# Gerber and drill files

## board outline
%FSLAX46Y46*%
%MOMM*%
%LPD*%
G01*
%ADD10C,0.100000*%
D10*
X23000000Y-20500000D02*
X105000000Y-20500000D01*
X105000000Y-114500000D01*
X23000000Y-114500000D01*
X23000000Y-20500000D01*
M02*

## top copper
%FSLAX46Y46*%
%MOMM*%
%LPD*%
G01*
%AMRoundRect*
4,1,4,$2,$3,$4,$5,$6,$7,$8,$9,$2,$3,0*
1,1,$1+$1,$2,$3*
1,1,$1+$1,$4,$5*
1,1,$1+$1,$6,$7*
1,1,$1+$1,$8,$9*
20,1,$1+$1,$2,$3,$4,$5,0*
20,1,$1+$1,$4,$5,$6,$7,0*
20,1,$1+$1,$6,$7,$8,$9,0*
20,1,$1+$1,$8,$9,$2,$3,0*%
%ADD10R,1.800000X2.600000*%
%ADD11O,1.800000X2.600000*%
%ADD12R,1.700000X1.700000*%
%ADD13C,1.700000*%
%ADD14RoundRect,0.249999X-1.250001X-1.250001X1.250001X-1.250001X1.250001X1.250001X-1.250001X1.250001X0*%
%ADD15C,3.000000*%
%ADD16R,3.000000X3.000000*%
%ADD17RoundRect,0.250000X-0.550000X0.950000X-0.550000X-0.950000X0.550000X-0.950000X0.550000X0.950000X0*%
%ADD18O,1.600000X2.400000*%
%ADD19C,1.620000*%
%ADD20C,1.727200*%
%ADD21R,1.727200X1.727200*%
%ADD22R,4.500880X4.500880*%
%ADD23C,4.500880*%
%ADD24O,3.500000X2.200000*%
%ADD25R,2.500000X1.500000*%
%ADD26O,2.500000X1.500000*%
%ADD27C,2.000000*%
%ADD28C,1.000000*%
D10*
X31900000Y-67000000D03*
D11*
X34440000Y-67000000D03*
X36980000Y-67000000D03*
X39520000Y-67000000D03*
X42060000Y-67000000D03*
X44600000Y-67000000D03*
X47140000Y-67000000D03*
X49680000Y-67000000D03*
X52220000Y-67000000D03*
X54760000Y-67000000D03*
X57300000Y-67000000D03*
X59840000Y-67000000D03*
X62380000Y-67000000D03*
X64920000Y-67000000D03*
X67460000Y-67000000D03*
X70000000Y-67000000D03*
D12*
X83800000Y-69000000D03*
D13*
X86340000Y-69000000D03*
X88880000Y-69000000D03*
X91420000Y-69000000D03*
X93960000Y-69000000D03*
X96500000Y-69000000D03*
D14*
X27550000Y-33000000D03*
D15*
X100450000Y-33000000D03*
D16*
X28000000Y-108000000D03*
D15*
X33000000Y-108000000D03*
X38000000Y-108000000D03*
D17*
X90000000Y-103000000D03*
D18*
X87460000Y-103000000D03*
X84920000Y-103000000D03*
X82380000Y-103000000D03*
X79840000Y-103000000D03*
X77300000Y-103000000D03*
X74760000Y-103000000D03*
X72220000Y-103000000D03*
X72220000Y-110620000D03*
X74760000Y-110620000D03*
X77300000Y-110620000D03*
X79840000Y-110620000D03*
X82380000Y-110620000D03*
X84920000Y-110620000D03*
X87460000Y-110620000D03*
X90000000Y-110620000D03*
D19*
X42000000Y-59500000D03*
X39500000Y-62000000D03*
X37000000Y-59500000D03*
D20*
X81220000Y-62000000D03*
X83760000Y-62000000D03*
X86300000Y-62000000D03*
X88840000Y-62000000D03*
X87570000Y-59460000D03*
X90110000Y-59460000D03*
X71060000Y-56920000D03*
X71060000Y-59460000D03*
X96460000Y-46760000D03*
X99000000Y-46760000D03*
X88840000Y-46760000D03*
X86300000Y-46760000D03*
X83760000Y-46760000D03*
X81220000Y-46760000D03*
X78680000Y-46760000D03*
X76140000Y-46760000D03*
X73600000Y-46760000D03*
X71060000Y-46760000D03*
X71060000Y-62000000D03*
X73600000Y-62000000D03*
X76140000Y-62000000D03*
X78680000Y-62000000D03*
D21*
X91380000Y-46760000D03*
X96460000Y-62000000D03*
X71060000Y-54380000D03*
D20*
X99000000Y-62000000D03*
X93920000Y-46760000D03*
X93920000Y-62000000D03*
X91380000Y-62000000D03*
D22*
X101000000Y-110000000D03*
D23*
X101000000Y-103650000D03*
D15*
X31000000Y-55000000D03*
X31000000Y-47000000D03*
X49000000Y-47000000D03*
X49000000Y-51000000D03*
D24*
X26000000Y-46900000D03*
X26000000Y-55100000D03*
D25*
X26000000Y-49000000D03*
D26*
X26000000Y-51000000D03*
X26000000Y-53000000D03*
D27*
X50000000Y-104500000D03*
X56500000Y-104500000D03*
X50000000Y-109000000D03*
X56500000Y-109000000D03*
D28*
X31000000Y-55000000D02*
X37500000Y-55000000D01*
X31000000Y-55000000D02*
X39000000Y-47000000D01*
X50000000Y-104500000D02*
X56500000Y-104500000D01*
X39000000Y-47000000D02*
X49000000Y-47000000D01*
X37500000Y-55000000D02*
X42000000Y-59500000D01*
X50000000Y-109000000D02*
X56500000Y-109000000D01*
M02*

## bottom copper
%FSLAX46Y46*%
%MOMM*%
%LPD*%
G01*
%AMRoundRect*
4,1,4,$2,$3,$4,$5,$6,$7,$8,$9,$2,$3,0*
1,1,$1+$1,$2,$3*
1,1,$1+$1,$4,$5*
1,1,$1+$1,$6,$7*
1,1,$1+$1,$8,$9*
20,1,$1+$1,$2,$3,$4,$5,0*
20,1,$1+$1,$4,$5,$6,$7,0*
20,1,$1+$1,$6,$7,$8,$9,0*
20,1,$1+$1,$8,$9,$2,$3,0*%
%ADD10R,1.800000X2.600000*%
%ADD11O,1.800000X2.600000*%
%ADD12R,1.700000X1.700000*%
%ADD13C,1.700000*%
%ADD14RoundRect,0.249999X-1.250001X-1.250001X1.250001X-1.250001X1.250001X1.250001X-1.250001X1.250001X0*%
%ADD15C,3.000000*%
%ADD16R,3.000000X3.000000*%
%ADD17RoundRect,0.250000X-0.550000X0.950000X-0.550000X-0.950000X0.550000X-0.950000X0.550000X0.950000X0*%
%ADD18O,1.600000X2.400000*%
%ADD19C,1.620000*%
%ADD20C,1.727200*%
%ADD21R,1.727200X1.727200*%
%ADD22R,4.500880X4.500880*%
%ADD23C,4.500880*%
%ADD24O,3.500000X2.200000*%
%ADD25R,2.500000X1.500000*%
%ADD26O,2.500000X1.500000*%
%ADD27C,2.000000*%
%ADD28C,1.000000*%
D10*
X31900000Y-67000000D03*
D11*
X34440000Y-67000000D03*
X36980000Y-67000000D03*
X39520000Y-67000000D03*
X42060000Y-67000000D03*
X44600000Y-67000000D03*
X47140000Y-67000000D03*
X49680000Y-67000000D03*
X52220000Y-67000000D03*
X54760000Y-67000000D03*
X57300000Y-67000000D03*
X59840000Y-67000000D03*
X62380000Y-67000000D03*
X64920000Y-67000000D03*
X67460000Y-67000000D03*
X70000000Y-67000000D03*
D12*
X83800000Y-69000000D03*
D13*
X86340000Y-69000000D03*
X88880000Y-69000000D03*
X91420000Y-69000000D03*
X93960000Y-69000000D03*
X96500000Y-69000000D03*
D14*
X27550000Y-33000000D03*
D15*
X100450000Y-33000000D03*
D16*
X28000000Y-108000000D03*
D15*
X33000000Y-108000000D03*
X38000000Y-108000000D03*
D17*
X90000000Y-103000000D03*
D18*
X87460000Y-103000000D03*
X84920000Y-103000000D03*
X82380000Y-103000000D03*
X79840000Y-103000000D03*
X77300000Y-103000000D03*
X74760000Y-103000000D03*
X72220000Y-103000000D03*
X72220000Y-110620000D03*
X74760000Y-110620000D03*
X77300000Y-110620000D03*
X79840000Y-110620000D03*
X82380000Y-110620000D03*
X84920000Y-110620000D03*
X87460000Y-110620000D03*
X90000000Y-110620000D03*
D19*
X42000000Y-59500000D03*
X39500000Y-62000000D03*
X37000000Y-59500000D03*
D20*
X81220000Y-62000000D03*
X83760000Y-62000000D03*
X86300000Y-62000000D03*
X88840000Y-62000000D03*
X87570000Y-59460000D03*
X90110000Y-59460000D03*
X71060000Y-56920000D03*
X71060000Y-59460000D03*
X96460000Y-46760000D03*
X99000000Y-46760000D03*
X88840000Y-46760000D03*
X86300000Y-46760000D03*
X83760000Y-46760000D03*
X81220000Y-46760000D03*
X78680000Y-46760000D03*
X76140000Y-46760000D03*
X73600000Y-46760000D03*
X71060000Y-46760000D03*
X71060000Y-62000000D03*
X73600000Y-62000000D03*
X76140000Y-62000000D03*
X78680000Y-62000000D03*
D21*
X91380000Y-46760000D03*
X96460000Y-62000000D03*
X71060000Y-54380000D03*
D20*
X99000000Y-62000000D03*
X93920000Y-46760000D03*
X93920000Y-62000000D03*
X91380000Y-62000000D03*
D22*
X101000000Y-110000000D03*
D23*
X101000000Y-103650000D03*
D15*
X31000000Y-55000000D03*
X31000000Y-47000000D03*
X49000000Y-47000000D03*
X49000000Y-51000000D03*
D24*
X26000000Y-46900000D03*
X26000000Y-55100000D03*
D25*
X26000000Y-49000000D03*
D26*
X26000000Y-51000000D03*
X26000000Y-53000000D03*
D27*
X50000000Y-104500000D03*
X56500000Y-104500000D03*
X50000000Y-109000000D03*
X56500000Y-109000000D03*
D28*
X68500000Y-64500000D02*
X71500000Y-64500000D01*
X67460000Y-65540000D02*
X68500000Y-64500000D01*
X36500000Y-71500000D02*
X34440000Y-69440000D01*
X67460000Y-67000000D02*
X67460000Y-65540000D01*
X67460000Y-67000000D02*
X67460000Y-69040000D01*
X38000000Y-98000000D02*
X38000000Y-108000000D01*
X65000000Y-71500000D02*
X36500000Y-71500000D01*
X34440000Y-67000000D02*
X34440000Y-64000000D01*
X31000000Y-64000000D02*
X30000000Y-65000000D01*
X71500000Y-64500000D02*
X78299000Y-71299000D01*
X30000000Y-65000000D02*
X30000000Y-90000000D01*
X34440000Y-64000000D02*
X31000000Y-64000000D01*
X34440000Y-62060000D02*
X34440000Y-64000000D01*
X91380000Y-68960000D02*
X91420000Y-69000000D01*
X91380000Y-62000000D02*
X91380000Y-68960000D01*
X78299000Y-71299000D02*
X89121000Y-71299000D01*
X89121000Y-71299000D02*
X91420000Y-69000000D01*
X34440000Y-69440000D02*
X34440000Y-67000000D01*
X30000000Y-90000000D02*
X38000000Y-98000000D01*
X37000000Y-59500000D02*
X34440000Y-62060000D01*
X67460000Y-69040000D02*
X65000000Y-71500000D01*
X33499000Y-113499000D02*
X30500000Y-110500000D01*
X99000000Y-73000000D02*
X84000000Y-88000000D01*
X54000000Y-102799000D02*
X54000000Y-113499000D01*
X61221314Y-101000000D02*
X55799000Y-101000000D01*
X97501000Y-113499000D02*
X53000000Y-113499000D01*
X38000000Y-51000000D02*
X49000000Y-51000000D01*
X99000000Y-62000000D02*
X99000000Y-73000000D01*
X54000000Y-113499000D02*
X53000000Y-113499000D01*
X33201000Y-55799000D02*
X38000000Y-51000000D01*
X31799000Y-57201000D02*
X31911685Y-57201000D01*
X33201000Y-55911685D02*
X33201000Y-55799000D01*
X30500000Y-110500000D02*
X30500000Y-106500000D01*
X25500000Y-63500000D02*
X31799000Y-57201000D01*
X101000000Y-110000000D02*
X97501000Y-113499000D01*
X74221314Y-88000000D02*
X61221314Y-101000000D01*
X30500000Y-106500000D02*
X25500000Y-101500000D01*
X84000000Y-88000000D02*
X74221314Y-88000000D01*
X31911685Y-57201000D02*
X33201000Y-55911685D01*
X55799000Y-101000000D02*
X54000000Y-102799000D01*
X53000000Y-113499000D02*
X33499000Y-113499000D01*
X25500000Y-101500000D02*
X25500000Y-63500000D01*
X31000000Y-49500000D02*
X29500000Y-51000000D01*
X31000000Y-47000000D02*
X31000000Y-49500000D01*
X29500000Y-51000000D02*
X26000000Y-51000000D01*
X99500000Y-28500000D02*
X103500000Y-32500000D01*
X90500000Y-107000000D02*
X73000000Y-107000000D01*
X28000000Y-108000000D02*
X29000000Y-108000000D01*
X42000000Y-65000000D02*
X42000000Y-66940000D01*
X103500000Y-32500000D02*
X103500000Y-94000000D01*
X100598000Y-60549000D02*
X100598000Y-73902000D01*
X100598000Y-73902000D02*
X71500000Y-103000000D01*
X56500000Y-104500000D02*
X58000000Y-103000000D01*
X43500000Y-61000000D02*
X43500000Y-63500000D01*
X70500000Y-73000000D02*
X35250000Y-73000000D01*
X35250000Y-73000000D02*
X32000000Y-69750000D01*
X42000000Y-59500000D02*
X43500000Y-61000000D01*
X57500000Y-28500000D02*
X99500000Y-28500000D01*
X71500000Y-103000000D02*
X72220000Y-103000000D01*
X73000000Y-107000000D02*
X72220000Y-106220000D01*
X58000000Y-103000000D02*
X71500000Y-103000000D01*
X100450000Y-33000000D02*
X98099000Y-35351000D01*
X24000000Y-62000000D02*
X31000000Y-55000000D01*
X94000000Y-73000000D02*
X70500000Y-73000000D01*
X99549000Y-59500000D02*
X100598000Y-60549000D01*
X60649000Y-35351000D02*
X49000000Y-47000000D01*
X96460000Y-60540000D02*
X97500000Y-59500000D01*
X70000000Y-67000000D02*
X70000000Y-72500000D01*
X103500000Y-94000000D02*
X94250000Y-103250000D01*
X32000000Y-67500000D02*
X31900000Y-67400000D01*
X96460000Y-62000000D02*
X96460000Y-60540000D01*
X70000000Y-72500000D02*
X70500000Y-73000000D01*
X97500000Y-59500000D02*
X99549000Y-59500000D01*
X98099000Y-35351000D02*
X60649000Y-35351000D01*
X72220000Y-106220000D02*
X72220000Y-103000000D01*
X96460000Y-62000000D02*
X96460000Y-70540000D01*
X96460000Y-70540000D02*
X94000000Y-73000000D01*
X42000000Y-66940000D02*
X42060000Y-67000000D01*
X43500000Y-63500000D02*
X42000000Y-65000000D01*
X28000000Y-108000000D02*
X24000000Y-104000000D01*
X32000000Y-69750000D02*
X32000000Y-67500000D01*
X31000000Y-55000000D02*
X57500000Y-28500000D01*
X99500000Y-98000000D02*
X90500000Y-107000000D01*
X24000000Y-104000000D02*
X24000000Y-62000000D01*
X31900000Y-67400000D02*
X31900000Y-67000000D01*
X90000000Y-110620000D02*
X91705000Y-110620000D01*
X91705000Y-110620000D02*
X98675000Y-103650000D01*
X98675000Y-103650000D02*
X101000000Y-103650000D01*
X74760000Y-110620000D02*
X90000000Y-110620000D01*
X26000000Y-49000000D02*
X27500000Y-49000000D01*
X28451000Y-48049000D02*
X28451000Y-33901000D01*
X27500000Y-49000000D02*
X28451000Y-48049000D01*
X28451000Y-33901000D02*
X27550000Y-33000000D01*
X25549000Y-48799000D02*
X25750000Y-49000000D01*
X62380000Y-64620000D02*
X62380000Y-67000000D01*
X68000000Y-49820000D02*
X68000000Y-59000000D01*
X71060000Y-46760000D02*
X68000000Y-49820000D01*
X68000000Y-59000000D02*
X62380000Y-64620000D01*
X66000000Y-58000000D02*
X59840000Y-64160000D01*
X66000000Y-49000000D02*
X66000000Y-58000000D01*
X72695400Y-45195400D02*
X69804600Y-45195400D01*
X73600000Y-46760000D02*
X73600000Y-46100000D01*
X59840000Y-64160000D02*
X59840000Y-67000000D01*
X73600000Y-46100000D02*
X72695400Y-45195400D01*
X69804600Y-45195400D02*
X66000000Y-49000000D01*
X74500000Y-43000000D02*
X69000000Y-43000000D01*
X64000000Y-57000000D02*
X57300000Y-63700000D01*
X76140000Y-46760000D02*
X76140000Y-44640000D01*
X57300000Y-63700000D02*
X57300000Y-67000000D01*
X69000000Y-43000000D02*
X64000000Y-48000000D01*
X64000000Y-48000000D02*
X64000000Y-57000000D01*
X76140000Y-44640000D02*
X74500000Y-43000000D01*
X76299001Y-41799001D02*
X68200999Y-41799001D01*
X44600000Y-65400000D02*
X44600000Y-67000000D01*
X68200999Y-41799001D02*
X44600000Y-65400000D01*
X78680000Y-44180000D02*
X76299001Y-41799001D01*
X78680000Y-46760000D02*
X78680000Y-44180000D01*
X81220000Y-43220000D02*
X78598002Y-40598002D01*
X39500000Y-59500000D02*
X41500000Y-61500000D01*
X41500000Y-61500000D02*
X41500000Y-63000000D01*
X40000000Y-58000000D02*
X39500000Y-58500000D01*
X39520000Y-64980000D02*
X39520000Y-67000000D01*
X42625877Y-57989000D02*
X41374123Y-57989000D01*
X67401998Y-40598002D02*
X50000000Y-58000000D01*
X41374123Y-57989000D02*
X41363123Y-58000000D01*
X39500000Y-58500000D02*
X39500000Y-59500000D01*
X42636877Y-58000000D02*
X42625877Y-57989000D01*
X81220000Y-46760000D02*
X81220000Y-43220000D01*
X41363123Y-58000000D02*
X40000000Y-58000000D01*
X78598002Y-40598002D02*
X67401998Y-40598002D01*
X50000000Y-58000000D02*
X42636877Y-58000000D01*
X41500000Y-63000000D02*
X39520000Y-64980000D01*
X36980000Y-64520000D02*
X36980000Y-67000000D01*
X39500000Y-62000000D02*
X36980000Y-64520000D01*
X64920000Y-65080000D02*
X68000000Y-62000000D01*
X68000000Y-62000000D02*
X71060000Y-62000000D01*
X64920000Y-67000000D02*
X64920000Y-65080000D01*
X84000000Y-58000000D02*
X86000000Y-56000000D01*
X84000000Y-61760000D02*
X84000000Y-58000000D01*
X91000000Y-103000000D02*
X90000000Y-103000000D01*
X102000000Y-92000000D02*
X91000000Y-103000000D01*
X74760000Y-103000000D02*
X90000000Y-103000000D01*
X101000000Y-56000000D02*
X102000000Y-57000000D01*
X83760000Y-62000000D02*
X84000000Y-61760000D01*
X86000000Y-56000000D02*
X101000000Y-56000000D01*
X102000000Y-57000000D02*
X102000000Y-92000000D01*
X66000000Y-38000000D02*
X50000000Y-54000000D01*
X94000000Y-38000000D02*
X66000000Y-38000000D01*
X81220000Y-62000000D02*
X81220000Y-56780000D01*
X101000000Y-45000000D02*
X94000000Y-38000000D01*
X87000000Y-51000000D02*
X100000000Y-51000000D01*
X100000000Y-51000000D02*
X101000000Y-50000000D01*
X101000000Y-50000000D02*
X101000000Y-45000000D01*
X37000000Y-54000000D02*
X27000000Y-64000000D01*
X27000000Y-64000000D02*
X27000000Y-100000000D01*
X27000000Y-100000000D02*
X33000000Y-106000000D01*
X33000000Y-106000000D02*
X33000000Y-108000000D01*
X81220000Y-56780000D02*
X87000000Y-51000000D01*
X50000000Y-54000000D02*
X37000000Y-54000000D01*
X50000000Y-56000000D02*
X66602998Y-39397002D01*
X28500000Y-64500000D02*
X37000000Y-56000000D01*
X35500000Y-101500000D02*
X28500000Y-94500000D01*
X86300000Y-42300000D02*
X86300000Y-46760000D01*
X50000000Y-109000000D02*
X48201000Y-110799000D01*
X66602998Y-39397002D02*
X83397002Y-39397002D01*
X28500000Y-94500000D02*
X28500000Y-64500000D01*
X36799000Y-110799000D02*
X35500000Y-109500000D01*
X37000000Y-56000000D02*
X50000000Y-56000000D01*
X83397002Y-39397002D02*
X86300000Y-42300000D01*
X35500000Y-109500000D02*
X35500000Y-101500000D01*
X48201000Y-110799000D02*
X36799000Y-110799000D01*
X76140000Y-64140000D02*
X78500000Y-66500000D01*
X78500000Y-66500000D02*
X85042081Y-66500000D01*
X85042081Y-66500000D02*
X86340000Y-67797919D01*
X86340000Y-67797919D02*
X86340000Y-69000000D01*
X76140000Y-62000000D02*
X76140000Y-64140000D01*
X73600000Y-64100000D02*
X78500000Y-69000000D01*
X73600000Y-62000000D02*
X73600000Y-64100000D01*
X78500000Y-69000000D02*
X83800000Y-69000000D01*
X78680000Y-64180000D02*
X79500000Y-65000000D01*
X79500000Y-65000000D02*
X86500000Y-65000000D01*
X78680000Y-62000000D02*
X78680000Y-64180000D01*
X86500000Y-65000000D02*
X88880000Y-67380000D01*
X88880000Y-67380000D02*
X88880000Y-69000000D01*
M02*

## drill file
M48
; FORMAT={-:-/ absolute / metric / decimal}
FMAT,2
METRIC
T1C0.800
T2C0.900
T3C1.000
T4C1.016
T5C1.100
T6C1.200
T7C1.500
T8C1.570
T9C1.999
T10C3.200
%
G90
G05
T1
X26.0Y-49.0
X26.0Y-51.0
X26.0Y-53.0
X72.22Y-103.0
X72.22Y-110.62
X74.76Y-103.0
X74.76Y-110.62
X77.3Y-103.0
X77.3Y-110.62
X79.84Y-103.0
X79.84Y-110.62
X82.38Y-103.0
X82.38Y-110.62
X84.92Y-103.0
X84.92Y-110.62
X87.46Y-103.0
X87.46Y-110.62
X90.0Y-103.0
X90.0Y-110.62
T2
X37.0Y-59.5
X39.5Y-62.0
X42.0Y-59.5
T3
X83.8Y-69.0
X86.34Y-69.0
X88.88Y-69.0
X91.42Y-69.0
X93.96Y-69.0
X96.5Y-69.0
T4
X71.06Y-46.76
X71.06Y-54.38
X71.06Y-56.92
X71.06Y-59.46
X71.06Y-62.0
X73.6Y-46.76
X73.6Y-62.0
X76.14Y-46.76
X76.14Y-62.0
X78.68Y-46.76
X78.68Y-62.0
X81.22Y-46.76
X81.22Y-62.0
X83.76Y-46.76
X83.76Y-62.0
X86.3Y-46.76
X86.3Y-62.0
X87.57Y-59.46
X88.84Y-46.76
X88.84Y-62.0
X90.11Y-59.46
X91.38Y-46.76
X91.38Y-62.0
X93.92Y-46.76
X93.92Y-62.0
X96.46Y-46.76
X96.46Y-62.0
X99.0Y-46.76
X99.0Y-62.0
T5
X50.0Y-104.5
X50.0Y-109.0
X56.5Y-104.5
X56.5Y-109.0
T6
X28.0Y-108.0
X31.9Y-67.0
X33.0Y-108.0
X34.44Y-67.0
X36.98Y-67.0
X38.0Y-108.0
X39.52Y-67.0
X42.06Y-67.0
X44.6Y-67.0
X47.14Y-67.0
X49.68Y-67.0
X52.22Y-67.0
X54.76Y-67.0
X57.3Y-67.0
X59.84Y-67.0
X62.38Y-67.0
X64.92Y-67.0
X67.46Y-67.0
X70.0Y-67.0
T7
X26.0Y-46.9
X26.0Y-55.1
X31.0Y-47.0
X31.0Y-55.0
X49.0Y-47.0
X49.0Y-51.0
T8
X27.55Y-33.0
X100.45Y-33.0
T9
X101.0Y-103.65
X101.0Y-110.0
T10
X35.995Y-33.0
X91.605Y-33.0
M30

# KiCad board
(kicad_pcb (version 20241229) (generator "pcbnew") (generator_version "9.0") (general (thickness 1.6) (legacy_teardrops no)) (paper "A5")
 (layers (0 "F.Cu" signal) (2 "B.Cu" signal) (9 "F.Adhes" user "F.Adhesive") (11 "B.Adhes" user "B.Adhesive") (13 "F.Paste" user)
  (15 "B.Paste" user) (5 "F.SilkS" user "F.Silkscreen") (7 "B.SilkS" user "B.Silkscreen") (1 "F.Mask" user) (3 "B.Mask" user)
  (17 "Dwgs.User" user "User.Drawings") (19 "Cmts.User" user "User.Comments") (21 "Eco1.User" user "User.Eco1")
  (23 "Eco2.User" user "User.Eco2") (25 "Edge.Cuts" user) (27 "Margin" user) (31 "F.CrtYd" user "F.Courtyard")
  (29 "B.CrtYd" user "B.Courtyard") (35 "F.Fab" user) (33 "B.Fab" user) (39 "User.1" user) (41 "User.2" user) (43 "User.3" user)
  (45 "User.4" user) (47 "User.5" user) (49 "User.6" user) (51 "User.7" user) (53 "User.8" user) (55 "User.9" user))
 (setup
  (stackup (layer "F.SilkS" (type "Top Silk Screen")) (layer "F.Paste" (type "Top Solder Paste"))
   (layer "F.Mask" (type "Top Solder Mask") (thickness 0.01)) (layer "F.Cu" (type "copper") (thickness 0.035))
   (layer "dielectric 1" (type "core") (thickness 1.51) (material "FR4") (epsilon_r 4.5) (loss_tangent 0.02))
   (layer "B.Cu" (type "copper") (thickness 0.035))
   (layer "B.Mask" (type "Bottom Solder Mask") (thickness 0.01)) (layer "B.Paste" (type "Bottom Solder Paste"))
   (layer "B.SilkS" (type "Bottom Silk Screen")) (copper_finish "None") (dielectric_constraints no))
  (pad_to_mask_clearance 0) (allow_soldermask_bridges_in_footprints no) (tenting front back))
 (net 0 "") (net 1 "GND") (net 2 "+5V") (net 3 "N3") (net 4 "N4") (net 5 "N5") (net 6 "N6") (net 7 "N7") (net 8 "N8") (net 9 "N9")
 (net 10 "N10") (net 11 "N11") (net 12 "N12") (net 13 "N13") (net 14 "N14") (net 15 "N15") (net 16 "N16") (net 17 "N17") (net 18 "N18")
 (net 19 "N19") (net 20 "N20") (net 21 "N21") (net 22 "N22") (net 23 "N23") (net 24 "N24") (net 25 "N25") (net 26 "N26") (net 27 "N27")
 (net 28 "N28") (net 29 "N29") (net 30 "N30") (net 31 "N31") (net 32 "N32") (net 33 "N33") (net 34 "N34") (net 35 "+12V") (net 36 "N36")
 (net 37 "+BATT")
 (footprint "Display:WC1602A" (layer "F.Cu") (at 31.9 67)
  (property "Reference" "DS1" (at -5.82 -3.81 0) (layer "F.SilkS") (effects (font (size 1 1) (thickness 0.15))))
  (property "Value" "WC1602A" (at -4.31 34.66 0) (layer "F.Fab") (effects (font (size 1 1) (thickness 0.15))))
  (pad "1" thru_hole rect (at 0 0) (size 1.8 2.6) (drill 1.2) (layers "*.Cu" "*.Mask") (remove_unused_layers no) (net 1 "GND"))
  (pad "2" thru_hole oval (at 2.54 0) (size 1.8 2.6) (drill 1.2) (layers "*.Cu" "*.Mask") (remove_unused_layers no) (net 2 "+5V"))
  (pad "3" thru_hole oval (at 5.08 0) (size 1.8 2.6) (drill 1.2) (layers "*.Cu" "*.Mask") (remove_unused_layers no) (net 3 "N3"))
  (pad "4" thru_hole oval (at 7.62 0) (size 1.8 2.6) (drill 1.2) (layers "*.Cu" "*.Mask") (remove_unused_layers no) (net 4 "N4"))
  (pad "5" thru_hole oval (at 10.16 0) (size 1.8 2.6) (drill 1.2) (layers "*.Cu" "*.Mask") (remove_unused_layers no) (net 1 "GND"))
  (pad "6" thru_hole oval (at 12.7 0) (size 1.8 2.6) (drill 1.2) (layers "*.Cu" "*.Mask") (remove_unused_layers no) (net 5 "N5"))
  (pad "7" thru_hole oval (at 15.24 0) (size 1.8 2.6) (drill 1.2) (layers "*.Cu" "*.Mask") (remove_unused_layers no) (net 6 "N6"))
  (pad "8" thru_hole oval (at 17.78 0) (size 1.8 2.6) (drill 1.2) (layers "*.Cu" "*.Mask") (remove_unused_layers no) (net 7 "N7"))
  (pad "9" thru_hole oval (at 20.32 0) (size 1.8 2.6) (drill 1.2) (layers "*.Cu" "*.Mask") (remove_unused_layers no) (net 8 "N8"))
  (pad "10" thru_hole oval (at 22.86 0) (size 1.8 2.6) (drill 1.2) (layers "*.Cu" "*.Mask") (remove_unused_layers no) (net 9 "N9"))
  (pad "11" thru_hole oval (at 25.4 0) (size 1.8 2.6) (drill 1.2) (layers "*.Cu" "*.Mask") (remove_unused_layers no) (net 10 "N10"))
  (pad "12" thru_hole oval (at 27.94 0) (size 1.8 2.6) (drill 1.2) (layers "*.Cu" "*.Mask") (remove_unused_layers no) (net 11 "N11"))
  (pad "13" thru_hole oval (at 30.48 0) (size 1.8 2.6) (drill 1.2) (layers "*.Cu" "*.Mask") (remove_unused_layers no) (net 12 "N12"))
  (pad "14" thru_hole oval (at 33.02 0) (size 1.8 2.6) (drill 1.2) (layers "*.Cu" "*.Mask") (remove_unused_layers no) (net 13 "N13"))
  (pad "15" thru_hole oval (at 35.56 0) (size 1.8 2.6) (drill 1.2) (layers "*.Cu" "*.Mask") (remove_unused_layers no) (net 2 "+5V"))
  (pad "16" thru_hole oval (at 38.1 0) (size 1.8 2.6) (drill 1.2) (layers "*.Cu" "*.Mask") (remove_unused_layers no) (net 1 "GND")))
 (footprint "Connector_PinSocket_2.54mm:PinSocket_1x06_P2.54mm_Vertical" (layer "F.Cu") (at 83.8 69 90)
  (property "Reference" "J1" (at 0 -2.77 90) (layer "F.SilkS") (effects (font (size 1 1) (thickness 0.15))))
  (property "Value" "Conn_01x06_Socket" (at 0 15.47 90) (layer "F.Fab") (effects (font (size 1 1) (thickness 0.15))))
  (pad "1" thru_hole rect (at 0 0 90) (size 1.7 1.7) (drill 1) (layers "*.Cu" "*.Mask") (remove_unused_layers no) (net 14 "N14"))
  (pad "2" thru_hole circle (at 0 2.54 90) (size 1.7 1.7) (drill 1) (layers "*.Cu" "*.Mask") (remove_unused_layers no) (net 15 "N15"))
  (pad "3" thru_hole circle (at 0 5.08 90) (size 1.7 1.7) (drill 1) (layers "*.Cu" "*.Mask") (remove_unused_layers no) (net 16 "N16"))
  (pad "4" thru_hole circle (at 0 7.62 90) (size 1.7 1.7) (drill 1) (layers "*.Cu" "*.Mask") (remove_unused_layers no) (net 2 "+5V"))
  (pad "5" thru_hole circle (at 0 10.16 90) (size 1.7 1.7) (drill 1) (layers "*.Cu" "*.Mask") (remove_unused_layers no) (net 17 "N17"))
  (pad "6" thru_hole circle (at 0 12.7 90) (size 1.7 1.7) (drill 1) (layers "*.Cu" "*.Mask") (remove_unused_layers no) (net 1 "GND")))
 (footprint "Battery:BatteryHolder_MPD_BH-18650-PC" (layer "F.Cu") (at 27.55 33)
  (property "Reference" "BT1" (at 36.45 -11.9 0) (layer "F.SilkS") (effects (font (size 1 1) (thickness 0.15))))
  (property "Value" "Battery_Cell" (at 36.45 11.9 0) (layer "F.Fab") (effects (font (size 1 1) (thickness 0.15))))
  (pad "" np_thru_hole circle (at 8.445 0) (size 3.2 3.2) (drill 3.2) (layers "*.Cu" "*.Mask"))
  (pad "" np_thru_hole circle (at 64.055 0) (size 3.2 3.2) (drill 3.2) (layers "*.Cu" "*.Mask"))
  (pad "1" thru_hole roundrect (at 0 0) (size 3 3) (drill 1.57) (layers "*.Cu" "*.Mask") (remove_unused_layers no)
   (roundrect_rratio 0.083333) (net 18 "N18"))
  (pad "2" thru_hole circle (at 72.9 0) (size 3 3) (drill 1.57) (layers "*.Cu" "*.Mask") (remove_unused_layers no) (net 1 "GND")))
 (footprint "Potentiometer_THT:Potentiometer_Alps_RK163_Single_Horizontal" (layer "F.Cu") (at 28 108 90)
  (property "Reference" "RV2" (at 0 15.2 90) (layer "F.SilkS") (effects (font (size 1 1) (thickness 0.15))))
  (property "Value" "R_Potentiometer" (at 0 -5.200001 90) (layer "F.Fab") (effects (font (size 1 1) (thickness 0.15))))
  (pad "1" thru_hole rect (at 0 0 270) (size 3 3) (drill 1.2) (layers "*.Cu" "*.Mask") (remove_unused_layers no) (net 1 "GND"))
  (pad "2" thru_hole circle (at 0 5 270) (size 3 3) (drill 1.2) (layers "*.Cu" "*.Mask") (remove_unused_layers no) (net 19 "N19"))
  (pad "3" thru_hole circle (at 0 10 270) (size 3 3) (drill 1.2) (layers "*.Cu" "*.Mask") (remove_unused_layers no) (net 2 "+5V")))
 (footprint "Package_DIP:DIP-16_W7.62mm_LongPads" (layer "F.Cu") (at 90 103 -90)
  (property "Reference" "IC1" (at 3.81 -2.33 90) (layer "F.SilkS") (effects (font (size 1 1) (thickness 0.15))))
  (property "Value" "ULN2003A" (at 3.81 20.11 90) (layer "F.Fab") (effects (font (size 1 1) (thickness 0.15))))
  (pad "1" thru_hole roundrect (at 0 0 270) (size 2.4 1.6) (drill 0.8) (layers "*.Cu" "*.Mask") (remove_unused_layers no)
   (roundrect_rratio 0.15625) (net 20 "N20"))
  (pad "2" thru_hole oval (at 0 2.54 270) (size 2.4 1.6) (drill 0.8) (layers "*.Cu" "*.Mask") (remove_unused_layers no) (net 20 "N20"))
  (pad "3" thru_hole oval (at 0 5.08 270) (size 2.4 1.6) (drill 0.8) (layers "*.Cu" "*.Mask") (remove_unused_layers no) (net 20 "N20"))
  (pad "4" thru_hole oval (at 0 7.62 270) (size 2.4 1.6) (drill 0.8) (layers "*.Cu" "*.Mask") (remove_unused_layers no) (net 20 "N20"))
  (pad "5" thru_hole oval (at 0 10.16 270) (size 2.4 1.6) (drill 0.8) (layers "*.Cu" "*.Mask") (remove_unused_layers no) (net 20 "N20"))
  (pad "6" thru_hole oval (at 0 12.7 270) (size 2.4 1.6) (drill 0.8) (layers "*.Cu" "*.Mask") (remove_unused_layers no) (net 20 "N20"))
  (pad "7" thru_hole oval (at 0 15.24 270) (size 2.4 1.6) (drill 0.8) (layers "*.Cu" "*.Mask") (remove_unused_layers no) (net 20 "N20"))
  (pad "8" thru_hole oval (at 0 17.78 270) (size 2.4 1.6) (drill 0.8) (layers "*.Cu" "*.Mask") (remove_unused_layers no) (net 1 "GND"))
  (pad "9" thru_hole oval (at 7.62 17.78 270) (size 2.4 1.6) (drill 0.8) (layers "*.Cu" "*.Mask") (remove_unused_layers no) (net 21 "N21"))
  (pad "10" thru_hole oval (at 7.62 15.24 270) (size 2.4 1.6) (drill 0.8) (layers "*.Cu" "*.Mask") (remove_unused_layers no) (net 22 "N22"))
  (pad "11" thru_hole oval (at 7.62 12.7 270) (size 2.4 1.6) (drill 0.8) (layers "*.Cu" "*.Mask") (remove_unused_layers no) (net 22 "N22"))
  (pad "12" thru_hole oval (at 7.62 10.16 270) (size 2.4 1.6) (drill 0.8) (layers "*.Cu" "*.Mask") (remove_unused_layers no) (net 22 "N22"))
  (pad "13" thru_hole oval (at 7.62 7.62 270) (size 2.4 1.6) (drill 0.8) (layers "*.Cu" "*.Mask") (remove_unused_layers no) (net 22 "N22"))
  (pad "14" thru_hole oval (at 7.62 5.08 270) (size 2.4 1.6) (drill 0.8) (layers "*.Cu" "*.Mask") (remove_unused_layers no) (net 22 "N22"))
  (pad "15" thru_hole oval (at 7.62 2.54 270) (size 2.4 1.6) (drill 0.8) (layers "*.Cu" "*.Mask") (remove_unused_layers no) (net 22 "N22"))
  (pad "16" thru_hole oval (at 7.62 0 270) (size 2.4 1.6) (drill 0.8) (layers "*.Cu" "*.Mask") (remove_unused_layers no) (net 22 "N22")))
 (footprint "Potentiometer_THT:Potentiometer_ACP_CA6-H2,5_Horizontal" (layer "F.Cu") (at 42 59.5 -90)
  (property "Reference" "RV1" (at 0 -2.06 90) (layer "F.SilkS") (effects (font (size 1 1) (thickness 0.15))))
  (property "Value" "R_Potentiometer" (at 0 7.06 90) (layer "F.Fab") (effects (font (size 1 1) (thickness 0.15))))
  (pad "1" thru_hole circle (at 0 0 270) (size 1.62 1.62) (drill 0.9) (layers "*.Cu" "*.Mask") (remove_unused_layers no) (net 1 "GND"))
  (pad "2" thru_hole circle (at 2.5 2.5 270) (size 1.62 1.62) (drill 0.9) (layers "*.Cu" "*.Mask") (remove_unused_layers no) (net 3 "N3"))
  (pad "3" thru_hole circle (at 0 5 270) (size 1.62 1.62) (drill 0.9) (layers "*.Cu" "*.Mask") (remove_unused_layers no) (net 2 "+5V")))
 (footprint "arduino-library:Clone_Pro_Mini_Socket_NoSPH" (layer "F.Cu") (at 86.3 54.38 -90)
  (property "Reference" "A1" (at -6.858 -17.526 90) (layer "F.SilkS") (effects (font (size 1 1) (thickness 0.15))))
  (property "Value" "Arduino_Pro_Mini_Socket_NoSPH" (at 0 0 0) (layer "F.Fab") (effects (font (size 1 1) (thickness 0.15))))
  (pad "A0" thru_hole circle (at 7.62 5.08 270) (size 1.7272 1.7272) (drill 1.016) (layers "*.Cu" "*.Mask") (remove_unused_layers no)
   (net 19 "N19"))
  (pad "A1" thru_hole circle (at 7.62 2.54 270) (size 1.7272 1.7272) (drill 1.016) (layers "*.Cu" "*.Mask") (remove_unused_layers no)
   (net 20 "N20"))
  (pad "A2" thru_hole circle (at 7.62 0 270) (size 1.7272 1.7272) (drill 1.016) (layers "*.Cu" "*.Mask") (remove_unused_layers no)
   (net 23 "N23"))
  (pad "A3" thru_hole circle (at 7.62 -2.54 270) (size 1.7272 1.7272) (drill 1.016) (layers "*.Cu" "*.Mask") (remove_unused_layers no)
   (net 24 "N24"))
  (pad "A4" thru_hole circle (at 5.08 -1.27 270) (size 1.7272 1.7272) (drill 1.016) (layers "*.Cu" "*.Mask") (remove_unused_layers no)
   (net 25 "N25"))
  (pad "A5" thru_hole circle (at 5.08 -3.81 270) (size 1.7272 1.7272) (drill 1.016) (layers "*.Cu" "*.Mask") (remove_unused_layers no)
   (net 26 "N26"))
  (pad "A6" thru_hole circle (at 2.54 15.24 270) (size 1.7272 1.7272) (drill 1.016) (layers "*.Cu" "*.Mask") (remove_unused_layers no)
   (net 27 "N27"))
  (pad "A7" thru_hole circle (at 5.08 15.24 270) (size 1.7272 1.7272) (drill 1.016) (layers "*.Cu" "*.Mask") (remove_unused_layers no)
   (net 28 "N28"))
  (pad "D0" thru_hole circle (at -7.62 -10.16 270) (size 1.7272 1.7272) (drill 1.016) (layers "*.Cu" "*.Mask") (remove_unused_layers no)
   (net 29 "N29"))
  (pad "D1" thru_hole circle (at -7.62 -12.7 270) (size 1.7272 1.7272) (drill 1.016) (layers "*.Cu" "*.Mask") (remove_unused_layers no)
   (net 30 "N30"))
  (pad "D2" thru_hole circle (at -7.62 -2.54 270) (size 1.7272 1.7272) (drill 1.016) (layers "*.Cu" "*.Mask") (remove_unused_layers no)
   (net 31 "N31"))
  (pad "D3" thru_hole circle (at -7.62 0 270) (size 1.7272 1.7272) (drill 1.016) (layers "*.Cu" "*.Mask") (remove_unused_layers no)
   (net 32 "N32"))
  (pad "D4" thru_hole circle (at -7.62 2.54 270) (size 1.7272 1.7272) (drill 1.016) (layers "*.Cu" "*.Mask") (remove_unused_layers no)
   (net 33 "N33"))
  (pad "D5" thru_hole circle (at -7.62 5.08 270) (size 1.7272 1.7272) (drill 1.016) (layers "*.Cu" "*.Mask") (remove_unused_layers no)
   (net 4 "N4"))
  (pad "D6" thru_hole circle (at -7.62 7.62 270) (size 1.7272 1.7272) (drill 1.016) (layers "*.Cu" "*.Mask") (remove_unused_layers no)
   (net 5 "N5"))
  (pad "D7" thru_hole circle (at -7.62 10.16 270) (size 1.7272 1.7272) (drill 1.016) (layers "*.Cu" "*.Mask") (remove_unused_layers no)
   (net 10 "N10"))
  (pad "D8" thru_hole circle (at -7.62 12.7 270) (size 1.7272 1.7272) (drill 1.016) (layers "*.Cu" "*.Mask") (remove_unused_layers no)
   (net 11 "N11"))
  (pad "D9" thru_hole circle (at -7.62 15.24 270) (size 1.7272 1.7272) (drill 1.016) (layers "*.Cu" "*.Mask") (remove_unused_layers no)
   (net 12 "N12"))
  (pad "D10" thru_hole circle (at 7.62 15.24 270) (size 1.7272 1.7272) (drill 1.016) (layers "*.Cu" "*.Mask") (remove_unused_layers no)
   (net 13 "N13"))
  (pad "D11" thru_hole circle (at 7.62 12.7 270) (size 1.7272 1.7272) (drill 1.016) (layers "*.Cu" "*.Mask") (remove_unused_layers no)
   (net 14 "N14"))
  (pad "D12" thru_hole circle (at 7.62 10.16 270) (size 1.7272 1.7272) (drill 1.016) (layers "*.Cu" "*.Mask") (remove_unused_layers no)
   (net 15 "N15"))
  (pad "D13" thru_hole circle (at 7.62 7.62 270) (size 1.7272 1.7272) (drill 1.016) (layers "*.Cu" "*.Mask") (remove_unused_layers no)
   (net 16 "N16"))
  (pad "GND1" thru_hole rect (at -7.62 -5.08 270) (size 1.7272 1.7272) (drill 1.016) (layers "*.Cu" "*.Mask") (remove_unused_layers no)
   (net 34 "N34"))
  (pad "GND2" thru_hole rect (at 7.62 -10.16 270) (size 1.7272 1.7272) (drill 1.016) (layers "*.Cu" "*.Mask") (remove_unused_layers no)
   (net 1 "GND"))
  (pad "GND3" thru_hole rect (at 0 15.24 270) (size 1.7272 1.7272) (drill 1.016) (layers "*.Cu" "*.Mask") (remove_unused_layers no))
  (pad "RAW" thru_hole circle (at 7.62 -12.7 270) (size 1.7272 1.7272) (drill 1.016) (layers "*.Cu" "*.Mask") (remove_unused_layers no)
   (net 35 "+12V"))
  (pad "RST1" thru_hole circle (at -7.62 -7.62 270) (size 1.7272 1.7272) (drill 1.016) (layers "*.Cu" "*.Mask") (remove_unused_layers no)
   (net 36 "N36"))
  (pad "RST2" thru_hole circle (at 7.62 -7.62 270) (size 1.7272 1.7272) (drill 1.016) (layers "*.Cu" "*.Mask") (remove_unused_layers no)
   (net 17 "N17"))
  (pad "Vcc1" thru_hole circle (at 7.62 -5.08 270) (size 1.7272 1.7272) (drill 1.016) (layers "*.Cu" "*.Mask") (remove_unused_layers no)
   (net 2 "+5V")))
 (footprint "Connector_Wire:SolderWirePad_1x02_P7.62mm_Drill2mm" (layer "F.Cu") (at 101 110 90)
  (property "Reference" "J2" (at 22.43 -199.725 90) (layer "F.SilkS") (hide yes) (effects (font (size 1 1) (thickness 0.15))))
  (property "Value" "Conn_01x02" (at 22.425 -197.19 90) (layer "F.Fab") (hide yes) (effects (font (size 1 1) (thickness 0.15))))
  (pad "1" thru_hole rect (at 0 0 90) (size 4.50088 4.50088) (drill 1.99898) (layers "*.Cu" "*.Mask") (remove_unused_layers no)
   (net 35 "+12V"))
  (pad "2" thru_hole circle (at 6.35 0 90) (size 4.50088 4.50088) (drill 1.99898) (layers "*.Cu" "*.Mask") (remove_unused_layers no)
   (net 22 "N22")))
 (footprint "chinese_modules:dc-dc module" (layer "F.Cu") (at 40 51)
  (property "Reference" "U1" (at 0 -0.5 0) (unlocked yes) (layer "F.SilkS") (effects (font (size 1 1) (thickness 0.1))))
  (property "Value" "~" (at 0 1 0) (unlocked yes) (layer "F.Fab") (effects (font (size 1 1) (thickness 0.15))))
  (pad "1" thru_hole circle (at -9 4) (size 3 3) (drill 1.5) (layers "*.Cu" "*.Mask") (remove_unused_layers no) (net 1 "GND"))
  (pad "2" thru_hole circle (at -9 -4) (size 3 3) (drill 1.5) (layers "*.Cu" "*.Mask") (remove_unused_layers no) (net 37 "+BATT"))
  (pad "3" thru_hole circle (at 9 -4) (size 3 3) (drill 1.5) (layers "*.Cu" "*.Mask") (remove_unused_layers no) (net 1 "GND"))
  (pad "4" thru_hole circle (at 9 0) (size 3 3) (drill 1.5) (layers "*.Cu" "*.Mask") (remove_unused_layers no) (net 35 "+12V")))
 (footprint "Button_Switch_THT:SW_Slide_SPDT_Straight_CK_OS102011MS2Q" (layer "F.Cu") (at 26 49 -90)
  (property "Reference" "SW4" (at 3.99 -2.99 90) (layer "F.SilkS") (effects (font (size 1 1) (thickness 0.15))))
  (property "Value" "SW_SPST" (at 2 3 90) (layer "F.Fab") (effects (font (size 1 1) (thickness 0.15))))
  (pad "" thru_hole oval (at -2.1 0 270) (size 2.2 3.5) (drill 1.5) (layers "*.Cu" "*.Mask") (remove_unused_layers no))
  (pad "" thru_hole oval (at 6.1 0 270) (size 2.2 3.5) (drill 1.5) (layers "*.Cu" "*.Mask") (remove_unused_layers no))
  (pad "1" thru_hole rect (at 0 0 270) (size 1.5 2.5) (drill 0.8) (layers "*.Cu" "*.Mask") (remove_unused_layers no) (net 18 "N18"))
  (pad "2" thru_hole oval (at 2 0 270) (size 1.5 2.5) (drill 0.8) (layers "*.Cu" "*.Mask") (remove_unused_layers no) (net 37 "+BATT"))
  (pad "3" thru_hole oval (at 4 0 270) (size 1.5 2.5) (drill 0.8) (layers "*.Cu" "*.Mask") (remove_unused_layers no)))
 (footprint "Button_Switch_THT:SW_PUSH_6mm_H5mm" (layer "F.Cu") (at 50 104.5)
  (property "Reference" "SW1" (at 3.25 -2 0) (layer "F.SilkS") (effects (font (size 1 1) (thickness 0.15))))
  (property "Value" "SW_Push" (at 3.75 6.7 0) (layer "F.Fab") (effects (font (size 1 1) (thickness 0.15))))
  (pad "1" thru_hole circle (at 0 0 90) (size 2 2) (drill 1.1) (layers "*.Cu" "*.Mask") (remove_unused_layers no) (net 1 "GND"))
  (pad "1" thru_hole circle (at 6.5 0 90) (size 2 2) (drill 1.1) (layers "*.Cu" "*.Mask") (remove_unused_layers no) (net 1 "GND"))
  (pad "2" thru_hole circle (at 0 4.5 90) (size 2 2) (drill 1.1) (layers "*.Cu" "*.Mask") (remove_unused_layers no) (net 32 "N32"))
  (pad "2" thru_hole circle (at 6.5 4.5 90) (size 2 2) (drill 1.1) (layers "*.Cu" "*.Mask") (remove_unused_layers no) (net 32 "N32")))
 (gr_rect (start 23 20.5) (end 105 114.5) (stroke (width 0.1) (type solid)) (fill no) (layer "Edge.Cuts"))
 (segment (start 68.5 64.5) (end 71.5 64.5) (width 1) (layer "B.Cu") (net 2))
 (segment (start 67.46 65.54) (end 68.5 64.5) (width 1) (layer "B.Cu") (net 2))
 (segment (start 36.5 71.5) (end 34.44 69.44) (width 1) (layer "B.Cu") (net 2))
 (segment (start 67.46 67) (end 67.46 65.54) (width 1) (layer "B.Cu") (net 2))
 (segment (start 67.46 67) (end 67.46 69.04) (width 1) (layer "B.Cu") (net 2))
 (segment (start 38 98) (end 38 108) (width 1) (layer "B.Cu") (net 2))
 (segment (start 65 71.5) (end 36.5 71.5) (width 1) (layer "B.Cu") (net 2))
 (segment (start 34.44 67) (end 34.44 64) (width 1) (layer "B.Cu") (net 2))
 (segment (start 31 64) (end 30 65) (width 1) (layer "B.Cu") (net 2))
 (segment (start 71.5 64.5) (end 78.299 71.299) (width 1) (layer "B.Cu") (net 2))
 (segment (start 30 65) (end 30 90) (width 1) (layer "B.Cu") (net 2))
 (segment (start 34.44 64) (end 31 64) (width 1) (layer "B.Cu") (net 2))
 (segment (start 34.44 62.06) (end 34.44 64) (width 1) (layer "B.Cu") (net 2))
 (segment (start 91.38 68.96) (end 91.42 69) (width 1) (layer "B.Cu") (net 2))
 (segment (start 91.38 62) (end 91.38 68.96) (width 1) (layer "B.Cu") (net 2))
 (segment (start 78.299 71.299) (end 89.121 71.299) (width 1) (layer "B.Cu") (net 2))
 (segment (start 89.121 71.299) (end 91.42 69) (width 1) (layer "B.Cu") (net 2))
 (segment (start 34.44 69.44) (end 34.44 67) (width 1) (layer "B.Cu") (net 2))
 (segment (start 30 90) (end 38 98) (width 1) (layer "B.Cu") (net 2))
 (segment (start 37 59.5) (end 34.44 62.06) (width 1) (layer "B.Cu") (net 2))
 (segment (start 67.46 69.04) (end 65 71.5) (width 1) (layer "B.Cu") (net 2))
 (segment (start 33.499 113.499) (end 30.5 110.5) (width 1) (layer "B.Cu") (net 35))
 (segment (start 99 73) (end 84 88) (width 1) (layer "B.Cu") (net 35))
 (segment (start 54 102.799) (end 54 113.499) (width 1) (layer "B.Cu") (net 35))
 (segment (start 61.221314 101) (end 55.799 101) (width 1) (layer "B.Cu") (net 35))
 (segment (start 97.501 113.499) (end 53 113.499) (width 1) (layer "B.Cu") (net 35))
 (segment (start 38 51) (end 49 51) (width 1) (layer "B.Cu") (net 35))
 (segment (start 99 62) (end 99 73) (width 1) (layer "B.Cu") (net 35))
 (segment (start 54 113.499) (end 53 113.499) (width 1) (layer "B.Cu") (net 35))
 (segment (start 33.201 55.799) (end 38 51) (width 1) (layer "B.Cu") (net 35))
 (segment (start 31.799 57.201) (end 31.911685 57.201) (width 1) (layer "B.Cu") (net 35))
 (segment (start 33.201 55.911685) (end 33.201 55.799) (width 1) (layer "B.Cu") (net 35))
 (segment (start 30.5 110.5) (end 30.5 106.5) (width 1) (layer "B.Cu") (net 35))
 (segment (start 25.5 63.5) (end 31.799 57.201) (width 1) (layer "B.Cu") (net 35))
 (segment (start 101 110) (end 97.501 113.499) (width 1) (layer "B.Cu") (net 35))
 (segment (start 74.221314 88) (end 61.221314 101) (width 1) (layer "B.Cu") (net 35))
 (segment (start 30.5 106.5) (end 25.5 101.5) (width 1) (layer "B.Cu") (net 35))
 (segment (start 84 88) (end 74.221314 88) (width 1) (layer "B.Cu") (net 35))
 (segment (start 31.911685 57.201) (end 33.201 55.911685) (width 1) (layer "B.Cu") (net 35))
 (segment (start 55.799 101) (end 54 102.799) (width 1) (layer "B.Cu") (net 35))
 (segment (start 53 113.499) (end 33.499 113.499) (width 1) (layer "B.Cu") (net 35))
 (segment (start 25.5 101.5) (end 25.5 63.5) (width 1) (layer "B.Cu") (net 35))
 (segment (start 31 49.5) (end 29.5 51) (width 1) (layer "B.Cu") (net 37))
 (segment (start 31 47) (end 31 49.5) (width 1) (layer "B.Cu") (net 37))
 (segment (start 29.5 51) (end 26 51) (width 1) (layer "B.Cu") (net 37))
 (segment (start 31 55) (end 37.5 55) (width 1) (layer "F.Cu") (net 1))
 (segment (start 31 55) (end 39 47) (width 1) (layer "F.Cu") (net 1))
 (segment (start 50 104.5) (end 56.5 104.5) (width 1) (layer "F.Cu") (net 1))
 (segment (start 39 47) (end 49 47) (width 1) (layer "F.Cu") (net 1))
 (segment (start 37.5 55) (end 42 59.5) (width 1) (layer "F.Cu") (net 1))
 (segment (start 99.5 28.5) (end 103.5 32.5) (width 1) (layer "B.Cu") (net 1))
 (segment (start 90.5 107) (end 73 107) (width 1) (layer "B.Cu") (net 1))
 (segment (start 28 108) (end 29 108) (width 1) (layer "B.Cu") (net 1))
 (segment (start 42 65) (end 42 66.94) (width 1) (layer "B.Cu") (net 1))
 (segment (start 103.5 32.5) (end 103.5 94) (width 1) (layer "B.Cu") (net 1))
 (segment (start 100.598 60.549) (end 100.598 73.902) (width 1) (layer "B.Cu") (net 1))
 (segment (start 100.598 73.902) (end 71.5 103) (width 1) (layer "B.Cu") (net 1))
 (segment (start 56.5 104.5) (end 58 103) (width 1) (layer "B.Cu") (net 1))
 (segment (start 43.5 61) (end 43.5 63.5) (width 1) (layer "B.Cu") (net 1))
 (segment (start 70.5 73) (end 35.25 73) (width 1) (layer "B.Cu") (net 1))
 (segment (start 35.25 73) (end 32 69.75) (width 1) (layer "B.Cu") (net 1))
 (segment (start 42 59.5) (end 43.5 61) (width 1) (layer "B.Cu") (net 1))
 (segment (start 57.5 28.5) (end 99.5 28.5) (width 1) (layer "B.Cu") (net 1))
 (segment (start 71.5 103) (end 72.22 103) (width 1) (layer "B.Cu") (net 1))
 (segment (start 73 107) (end 72.22 106.22) (width 1) (layer "B.Cu") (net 1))
 (segment (start 58 103) (end 71.5 103) (width 1) (layer "B.Cu") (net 1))
 (segment (start 100.45 33) (end 98.099 35.351) (width 1) (layer "B.Cu") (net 1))
 (segment (start 24 62) (end 31 55) (width 1) (layer "B.Cu") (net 1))
 (segment (start 94 73) (end 70.5 73) (width 1) (layer "B.Cu") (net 1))
 (segment (start 99.549 59.5) (end 100.598 60.549) (width 1) (layer "B.Cu") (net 1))
 (segment (start 60.649 35.351) (end 49 47) (width 1) (layer "B.Cu") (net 1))
 (segment (start 96.46 60.54) (end 97.5 59.5) (width 1) (layer "B.Cu") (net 1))
 (segment (start 70 67) (end 70 72.5) (width 1) (layer "B.Cu") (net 1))
 (segment (start 103.5 94) (end 94.25 103.25) (width 1) (layer "B.Cu") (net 1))
 (segment (start 32 67.5) (end 31.9 67.4) (width 1) (layer "B.Cu") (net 1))
 (segment (start 96.46 62) (end 96.46 60.54) (width 1) (layer "B.Cu") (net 1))
 (segment (start 70 72.5) (end 70.5 73) (width 1) (layer "B.Cu") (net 1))
 (segment (start 97.5 59.5) (end 99.549 59.5) (width 1) (layer "B.Cu") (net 1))
 (segment (start 98.099 35.351) (end 60.649 35.351) (width 1) (layer "B.Cu") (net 1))
 (segment (start 72.22 106.22) (end 72.22 103) (width 1) (layer "B.Cu") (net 1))
 (segment (start 96.46 62) (end 96.46 70.54) (width 1) (layer "B.Cu") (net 1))
 (segment (start 96.46 70.54) (end 94 73) (width 1) (layer "B.Cu") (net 1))
 (segment (start 42 66.94) (end 42.06 67) (width 1) (layer "B.Cu") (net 1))
 (segment (start 43.5 63.5) (end 42 65) (width 1) (layer "B.Cu") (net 1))
 (segment (start 28 108) (end 24 104) (width 1) (layer "B.Cu") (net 1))
 (segment (start 32 69.75) (end 32 67.5) (width 1) (layer "B.Cu") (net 1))
 (segment (start 31 55) (end 57.5 28.5) (width 1) (layer "B.Cu") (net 1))
 (segment (start 99.5 98) (end 90.5 107) (width 1) (layer "B.Cu") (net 1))
 (segment (start 24 104) (end 24 62) (width 1) (layer "B.Cu") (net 1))
 (segment (start 31.9 67.4) (end 31.9 67) (width 1) (layer "B.Cu") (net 1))
 (segment (start 90 110.62) (end 91.705 110.62) (width 1) (layer "B.Cu") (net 22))
 (segment (start 91.705 110.62) (end 98.675 103.65) (width 1) (layer "B.Cu") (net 22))
 (segment (start 98.675 103.65) (end 101 103.65) (width 1) (layer "B.Cu") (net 22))
 (segment (start 74.76 110.62) (end 90 110.62) (width 1) (layer "B.Cu") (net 22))
 (segment (start 26 49) (end 27.5 49) (width 1) (layer "B.Cu") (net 18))
 (segment (start 28.451 48.049) (end 28.451 33.901) (width 1) (layer "B.Cu") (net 18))
 (segment (start 27.5 49) (end 28.451 48.049) (width 1) (layer "B.Cu") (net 18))
 (segment (start 28.451 33.901) (end 27.55 33) (width 1) (layer "B.Cu") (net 18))
 (segment (start 25.549 48.799) (end 25.75 49) (width 1) (layer "B.Cu") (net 18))
 (segment (start 62.38 64.62) (end 62.38 67) (width 1) (layer "B.Cu") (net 12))
 (segment (start 68 49.82) (end 68 59) (width 1) (layer "B.Cu") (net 12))
 (segment (start 71.06 46.76) (end 68 49.82) (width 1) (layer "B.Cu") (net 12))
 (segment (start 68 59) (end 62.38 64.62) (width 1) (layer "B.Cu") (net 12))
 (segment (start 66 58) (end 59.84 64.16) (width 1) (layer "B.Cu") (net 11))
 (segment (start 66 49) (end 66 58) (width 1) (layer "B.Cu") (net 11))
 (segment (start 72.6954 45.1954) (end 69.8046 45.1954) (width 1) (layer "B.Cu") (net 11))
 (segment (start 73.6 46.76) (end 73.6 46.1) (width 1) (layer "B.Cu") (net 11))
 (segment (start 59.84 64.16) (end 59.84 67) (width 1) (layer "B.Cu") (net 11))
 (segment (start 73.6 46.1) (end 72.6954 45.1954) (width 1) (layer "B.Cu") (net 11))
 (segment (start 69.8046 45.1954) (end 66 49) (width 1) (layer "B.Cu") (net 11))
 (segment (start 74.5 43) (end 69 43) (width 1) (layer "B.Cu") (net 10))
 (segment (start 64 57) (end 57.3 63.7) (width 1) (layer "B.Cu") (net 10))
 (segment (start 76.14 46.76) (end 76.14 44.64) (width 1) (layer "B.Cu") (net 10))
 (segment (start 57.3 63.7) (end 57.3 67) (width 1) (layer "B.Cu") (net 10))
 (segment (start 69 43) (end 64 48) (width 1) (layer "B.Cu") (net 10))
 (segment (start 64 48) (end 64 57) (width 1) (layer "B.Cu") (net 10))
 (segment (start 76.14 44.64) (end 74.5 43) (width 1) (layer "B.Cu") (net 10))
 (segment (start 76.299001 41.799001) (end 68.200999 41.799001) (width 1) (layer "B.Cu") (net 5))
 (segment (start 44.6 65.4) (end 44.6 67) (width 1) (layer "B.Cu") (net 5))
 (segment (start 68.200999 41.799001) (end 44.6 65.4) (width 1) (layer "B.Cu") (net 5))
 (segment (start 78.68 44.18) (end 76.299001 41.799001) (width 1) (layer "B.Cu") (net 5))
 (segment (start 78.68 46.76) (end 78.68 44.18) (width 1) (layer "B.Cu") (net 5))
 (segment (start 81.22 43.22) (end 78.598002 40.598002) (width 1) (layer "B.Cu") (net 4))
 (segment (start 39.5 59.5) (end 41.5 61.5) (width 1) (layer "B.Cu") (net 4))
 (segment (start 41.5 61.5) (end 41.5 63) (width 1) (layer "B.Cu") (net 4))
 (segment (start 40 58) (end 39.5 58.5) (width 1) (layer "B.Cu") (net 4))
 (segment (start 39.52 64.98) (end 39.52 67) (width 1) (layer "B.Cu") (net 4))
 (segment (start 42.625877 57.989) (end 41.374123 57.989) (width 1) (layer "B.Cu") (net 4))
 (segment (start 67.401998 40.598002) (end 50 58) (width 1) (layer "B.Cu") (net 4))
 (segment (start 41.374123 57.989) (end 41.363123 58) (width 1) (layer "B.Cu") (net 4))
 (segment (start 39.5 58.5) (end 39.5 59.5) (width 1) (layer "B.Cu") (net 4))
 (segment (start 42.636877 58) (end 42.625877 57.989) (width 1) (layer "B.Cu") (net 4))
 (segment (start 81.22 46.76) (end 81.22 43.22) (width 1) (layer "B.Cu") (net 4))
 (segment (start 41.363123 58) (end 40 58) (width 1) (layer "B.Cu") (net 4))
 (segment (start 78.598002 40.598002) (end 67.401998 40.598002) (width 1) (layer "B.Cu") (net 4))
 (segment (start 50 58) (end 42.636877 58) (width 1) (layer "B.Cu") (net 4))
 (segment (start 41.5 63) (end 39.52 64.98) (width 1) (layer "B.Cu") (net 4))
 (segment (start 36.98 64.52) (end 36.98 67) (width 1) (layer "B.Cu") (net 3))
 (segment (start 39.5 62) (end 36.98 64.52) (width 1) (layer "B.Cu") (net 3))
 (segment (start 64.92 65.08) (end 68 62) (width 1) (layer "B.Cu") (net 13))
 (segment (start 68 62) (end 71.06 62) (width 1) (layer "B.Cu") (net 13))
 (segment (start 64.92 67) (end 64.92 65.08) (width 1) (layer "B.Cu") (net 13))
 (segment (start 84 58) (end 86 56) (width 1) (layer "B.Cu") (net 20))
 (segment (start 84 61.76) (end 84 58) (width 1) (layer "B.Cu") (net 20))
 (segment (start 91 103) (end 90 103) (width 1) (layer "B.Cu") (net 20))
 (segment (start 102 92) (end 91 103) (width 1) (layer "B.Cu") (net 20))
 (segment (start 74.76 103) (end 90 103) (width 1) (layer "B.Cu") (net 20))
 (segment (start 101 56) (end 102 57) (width 1) (layer "B.Cu") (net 20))
 (segment (start 83.76 62) (end 84 61.76) (width 1) (layer "B.Cu") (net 20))
 (segment (start 86 56) (end 101 56) (width 1) (layer "B.Cu") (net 20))
 (segment (start 102 57) (end 102 92) (width 1) (layer "B.Cu") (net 20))
 (segment (start 66 38) (end 50 54) (width 1) (layer "B.Cu") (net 19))
 (segment (start 94 38) (end 66 38) (width 1) (layer "B.Cu") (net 19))
 (segment (start 81.22 62) (end 81.22 56.78) (width 1) (layer "B.Cu") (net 19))
 (segment (start 101 45) (end 94 38) (width 1) (layer "B.Cu") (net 19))
 (segment (start 87 51) (end 100 51) (width 1) (layer "B.Cu") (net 19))
 (segment (start 100 51) (end 101 50) (width 1) (layer "B.Cu") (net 19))
 (segment (start 101 50) (end 101 45) (width 1) (layer "B.Cu") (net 19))
 (segment (start 37 54) (end 27 64) (width 1) (layer "B.Cu") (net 19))
 (segment (start 27 64) (end 27 100) (width 1) (layer "B.Cu") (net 19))
 (segment (start 27 100) (end 33 106) (width 1) (layer "B.Cu") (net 19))
 (segment (start 33 106) (end 33 108) (width 1) (layer "B.Cu") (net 19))
 (segment (start 81.22 56.78) (end 87 51) (width 1) (layer "B.Cu") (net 19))
 (segment (start 50 54) (end 37 54) (width 1) (layer "B.Cu") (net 19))
 (segment (start 50 109) (end 56.5 109) (width 1) (layer "F.Cu") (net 32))
 (segment (start 50 56) (end 66.602998 39.397002) (width 1) (layer "B.Cu") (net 32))
 (segment (start 28.5 64.5) (end 37 56) (width 1) (layer "B.Cu") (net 32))
 (segment (start 35.5 101.5) (end 28.5 94.5) (width 1) (layer "B.Cu") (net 32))
 (segment (start 86.3 42.3) (end 86.3 46.76) (width 1) (layer "B.Cu") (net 32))
 (segment (start 50 109) (end 48.201 110.799) (width 1) (layer "B.Cu") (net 32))
 (segment (start 66.602998 39.397002) (end 83.397002 39.397002) (width 1) (layer "B.Cu") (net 32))
 (segment (start 28.5 94.5) (end 28.5 64.5) (width 1) (layer "B.Cu") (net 32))
 (segment (start 36.799 110.799) (end 35.5 109.5) (width 1) (layer "B.Cu") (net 32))
 (segment (start 37 56) (end 50 56) (width 1) (layer "B.Cu") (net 32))
 (segment (start 83.397002 39.397002) (end 86.3 42.3) (width 1) (layer "B.Cu") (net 32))
 (segment (start 35.5 109.5) (end 35.5 101.5) (width 1) (layer "B.Cu") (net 32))
 (segment (start 48.201 110.799) (end 36.799 110.799) (width 1) (layer "B.Cu") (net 32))
 (segment (start 76.14 64.14) (end 78.5 66.5) (width 1) (layer "B.Cu") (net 15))
 (segment (start 78.5 66.5) (end 85.042081 66.5) (width 1) (layer "B.Cu") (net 15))
 (segment (start 85.042081 66.5) (end 86.34 67.797919) (width 1) (layer "B.Cu") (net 15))
 (segment (start 86.34 67.797919) (end 86.34 69) (width 1) (layer "B.Cu") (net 15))
 (segment (start 76.14 62) (end 76.14 64.14) (width 1) (layer "B.Cu") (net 15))
 (segment (start 73.6 64.1) (end 78.5 69) (width 1) (layer "B.Cu") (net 14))
 (segment (start 73.6 62) (end 73.6 64.1) (width 1) (layer "B.Cu") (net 14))
 (segment (start 78.5 69) (end 83.8 69) (width 1) (layer "B.Cu") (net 14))
 (segment (start 78.68 64.18) (end 79.5 65) (width 1) (layer "B.Cu") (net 16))
 (segment (start 79.5 65) (end 86.5 65) (width 1) (layer "B.Cu") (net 16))
 (segment (start 78.68 62) (end 78.68 64.18) (width 1) (layer "B.Cu") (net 16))
 (segment (start 86.5 65) (end 88.88 67.38) (width 1) (layer "B.Cu") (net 16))
 (segment (start 88.88 67.38) (end 88.88 69) (width 1) (layer "B.Cu") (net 16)))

